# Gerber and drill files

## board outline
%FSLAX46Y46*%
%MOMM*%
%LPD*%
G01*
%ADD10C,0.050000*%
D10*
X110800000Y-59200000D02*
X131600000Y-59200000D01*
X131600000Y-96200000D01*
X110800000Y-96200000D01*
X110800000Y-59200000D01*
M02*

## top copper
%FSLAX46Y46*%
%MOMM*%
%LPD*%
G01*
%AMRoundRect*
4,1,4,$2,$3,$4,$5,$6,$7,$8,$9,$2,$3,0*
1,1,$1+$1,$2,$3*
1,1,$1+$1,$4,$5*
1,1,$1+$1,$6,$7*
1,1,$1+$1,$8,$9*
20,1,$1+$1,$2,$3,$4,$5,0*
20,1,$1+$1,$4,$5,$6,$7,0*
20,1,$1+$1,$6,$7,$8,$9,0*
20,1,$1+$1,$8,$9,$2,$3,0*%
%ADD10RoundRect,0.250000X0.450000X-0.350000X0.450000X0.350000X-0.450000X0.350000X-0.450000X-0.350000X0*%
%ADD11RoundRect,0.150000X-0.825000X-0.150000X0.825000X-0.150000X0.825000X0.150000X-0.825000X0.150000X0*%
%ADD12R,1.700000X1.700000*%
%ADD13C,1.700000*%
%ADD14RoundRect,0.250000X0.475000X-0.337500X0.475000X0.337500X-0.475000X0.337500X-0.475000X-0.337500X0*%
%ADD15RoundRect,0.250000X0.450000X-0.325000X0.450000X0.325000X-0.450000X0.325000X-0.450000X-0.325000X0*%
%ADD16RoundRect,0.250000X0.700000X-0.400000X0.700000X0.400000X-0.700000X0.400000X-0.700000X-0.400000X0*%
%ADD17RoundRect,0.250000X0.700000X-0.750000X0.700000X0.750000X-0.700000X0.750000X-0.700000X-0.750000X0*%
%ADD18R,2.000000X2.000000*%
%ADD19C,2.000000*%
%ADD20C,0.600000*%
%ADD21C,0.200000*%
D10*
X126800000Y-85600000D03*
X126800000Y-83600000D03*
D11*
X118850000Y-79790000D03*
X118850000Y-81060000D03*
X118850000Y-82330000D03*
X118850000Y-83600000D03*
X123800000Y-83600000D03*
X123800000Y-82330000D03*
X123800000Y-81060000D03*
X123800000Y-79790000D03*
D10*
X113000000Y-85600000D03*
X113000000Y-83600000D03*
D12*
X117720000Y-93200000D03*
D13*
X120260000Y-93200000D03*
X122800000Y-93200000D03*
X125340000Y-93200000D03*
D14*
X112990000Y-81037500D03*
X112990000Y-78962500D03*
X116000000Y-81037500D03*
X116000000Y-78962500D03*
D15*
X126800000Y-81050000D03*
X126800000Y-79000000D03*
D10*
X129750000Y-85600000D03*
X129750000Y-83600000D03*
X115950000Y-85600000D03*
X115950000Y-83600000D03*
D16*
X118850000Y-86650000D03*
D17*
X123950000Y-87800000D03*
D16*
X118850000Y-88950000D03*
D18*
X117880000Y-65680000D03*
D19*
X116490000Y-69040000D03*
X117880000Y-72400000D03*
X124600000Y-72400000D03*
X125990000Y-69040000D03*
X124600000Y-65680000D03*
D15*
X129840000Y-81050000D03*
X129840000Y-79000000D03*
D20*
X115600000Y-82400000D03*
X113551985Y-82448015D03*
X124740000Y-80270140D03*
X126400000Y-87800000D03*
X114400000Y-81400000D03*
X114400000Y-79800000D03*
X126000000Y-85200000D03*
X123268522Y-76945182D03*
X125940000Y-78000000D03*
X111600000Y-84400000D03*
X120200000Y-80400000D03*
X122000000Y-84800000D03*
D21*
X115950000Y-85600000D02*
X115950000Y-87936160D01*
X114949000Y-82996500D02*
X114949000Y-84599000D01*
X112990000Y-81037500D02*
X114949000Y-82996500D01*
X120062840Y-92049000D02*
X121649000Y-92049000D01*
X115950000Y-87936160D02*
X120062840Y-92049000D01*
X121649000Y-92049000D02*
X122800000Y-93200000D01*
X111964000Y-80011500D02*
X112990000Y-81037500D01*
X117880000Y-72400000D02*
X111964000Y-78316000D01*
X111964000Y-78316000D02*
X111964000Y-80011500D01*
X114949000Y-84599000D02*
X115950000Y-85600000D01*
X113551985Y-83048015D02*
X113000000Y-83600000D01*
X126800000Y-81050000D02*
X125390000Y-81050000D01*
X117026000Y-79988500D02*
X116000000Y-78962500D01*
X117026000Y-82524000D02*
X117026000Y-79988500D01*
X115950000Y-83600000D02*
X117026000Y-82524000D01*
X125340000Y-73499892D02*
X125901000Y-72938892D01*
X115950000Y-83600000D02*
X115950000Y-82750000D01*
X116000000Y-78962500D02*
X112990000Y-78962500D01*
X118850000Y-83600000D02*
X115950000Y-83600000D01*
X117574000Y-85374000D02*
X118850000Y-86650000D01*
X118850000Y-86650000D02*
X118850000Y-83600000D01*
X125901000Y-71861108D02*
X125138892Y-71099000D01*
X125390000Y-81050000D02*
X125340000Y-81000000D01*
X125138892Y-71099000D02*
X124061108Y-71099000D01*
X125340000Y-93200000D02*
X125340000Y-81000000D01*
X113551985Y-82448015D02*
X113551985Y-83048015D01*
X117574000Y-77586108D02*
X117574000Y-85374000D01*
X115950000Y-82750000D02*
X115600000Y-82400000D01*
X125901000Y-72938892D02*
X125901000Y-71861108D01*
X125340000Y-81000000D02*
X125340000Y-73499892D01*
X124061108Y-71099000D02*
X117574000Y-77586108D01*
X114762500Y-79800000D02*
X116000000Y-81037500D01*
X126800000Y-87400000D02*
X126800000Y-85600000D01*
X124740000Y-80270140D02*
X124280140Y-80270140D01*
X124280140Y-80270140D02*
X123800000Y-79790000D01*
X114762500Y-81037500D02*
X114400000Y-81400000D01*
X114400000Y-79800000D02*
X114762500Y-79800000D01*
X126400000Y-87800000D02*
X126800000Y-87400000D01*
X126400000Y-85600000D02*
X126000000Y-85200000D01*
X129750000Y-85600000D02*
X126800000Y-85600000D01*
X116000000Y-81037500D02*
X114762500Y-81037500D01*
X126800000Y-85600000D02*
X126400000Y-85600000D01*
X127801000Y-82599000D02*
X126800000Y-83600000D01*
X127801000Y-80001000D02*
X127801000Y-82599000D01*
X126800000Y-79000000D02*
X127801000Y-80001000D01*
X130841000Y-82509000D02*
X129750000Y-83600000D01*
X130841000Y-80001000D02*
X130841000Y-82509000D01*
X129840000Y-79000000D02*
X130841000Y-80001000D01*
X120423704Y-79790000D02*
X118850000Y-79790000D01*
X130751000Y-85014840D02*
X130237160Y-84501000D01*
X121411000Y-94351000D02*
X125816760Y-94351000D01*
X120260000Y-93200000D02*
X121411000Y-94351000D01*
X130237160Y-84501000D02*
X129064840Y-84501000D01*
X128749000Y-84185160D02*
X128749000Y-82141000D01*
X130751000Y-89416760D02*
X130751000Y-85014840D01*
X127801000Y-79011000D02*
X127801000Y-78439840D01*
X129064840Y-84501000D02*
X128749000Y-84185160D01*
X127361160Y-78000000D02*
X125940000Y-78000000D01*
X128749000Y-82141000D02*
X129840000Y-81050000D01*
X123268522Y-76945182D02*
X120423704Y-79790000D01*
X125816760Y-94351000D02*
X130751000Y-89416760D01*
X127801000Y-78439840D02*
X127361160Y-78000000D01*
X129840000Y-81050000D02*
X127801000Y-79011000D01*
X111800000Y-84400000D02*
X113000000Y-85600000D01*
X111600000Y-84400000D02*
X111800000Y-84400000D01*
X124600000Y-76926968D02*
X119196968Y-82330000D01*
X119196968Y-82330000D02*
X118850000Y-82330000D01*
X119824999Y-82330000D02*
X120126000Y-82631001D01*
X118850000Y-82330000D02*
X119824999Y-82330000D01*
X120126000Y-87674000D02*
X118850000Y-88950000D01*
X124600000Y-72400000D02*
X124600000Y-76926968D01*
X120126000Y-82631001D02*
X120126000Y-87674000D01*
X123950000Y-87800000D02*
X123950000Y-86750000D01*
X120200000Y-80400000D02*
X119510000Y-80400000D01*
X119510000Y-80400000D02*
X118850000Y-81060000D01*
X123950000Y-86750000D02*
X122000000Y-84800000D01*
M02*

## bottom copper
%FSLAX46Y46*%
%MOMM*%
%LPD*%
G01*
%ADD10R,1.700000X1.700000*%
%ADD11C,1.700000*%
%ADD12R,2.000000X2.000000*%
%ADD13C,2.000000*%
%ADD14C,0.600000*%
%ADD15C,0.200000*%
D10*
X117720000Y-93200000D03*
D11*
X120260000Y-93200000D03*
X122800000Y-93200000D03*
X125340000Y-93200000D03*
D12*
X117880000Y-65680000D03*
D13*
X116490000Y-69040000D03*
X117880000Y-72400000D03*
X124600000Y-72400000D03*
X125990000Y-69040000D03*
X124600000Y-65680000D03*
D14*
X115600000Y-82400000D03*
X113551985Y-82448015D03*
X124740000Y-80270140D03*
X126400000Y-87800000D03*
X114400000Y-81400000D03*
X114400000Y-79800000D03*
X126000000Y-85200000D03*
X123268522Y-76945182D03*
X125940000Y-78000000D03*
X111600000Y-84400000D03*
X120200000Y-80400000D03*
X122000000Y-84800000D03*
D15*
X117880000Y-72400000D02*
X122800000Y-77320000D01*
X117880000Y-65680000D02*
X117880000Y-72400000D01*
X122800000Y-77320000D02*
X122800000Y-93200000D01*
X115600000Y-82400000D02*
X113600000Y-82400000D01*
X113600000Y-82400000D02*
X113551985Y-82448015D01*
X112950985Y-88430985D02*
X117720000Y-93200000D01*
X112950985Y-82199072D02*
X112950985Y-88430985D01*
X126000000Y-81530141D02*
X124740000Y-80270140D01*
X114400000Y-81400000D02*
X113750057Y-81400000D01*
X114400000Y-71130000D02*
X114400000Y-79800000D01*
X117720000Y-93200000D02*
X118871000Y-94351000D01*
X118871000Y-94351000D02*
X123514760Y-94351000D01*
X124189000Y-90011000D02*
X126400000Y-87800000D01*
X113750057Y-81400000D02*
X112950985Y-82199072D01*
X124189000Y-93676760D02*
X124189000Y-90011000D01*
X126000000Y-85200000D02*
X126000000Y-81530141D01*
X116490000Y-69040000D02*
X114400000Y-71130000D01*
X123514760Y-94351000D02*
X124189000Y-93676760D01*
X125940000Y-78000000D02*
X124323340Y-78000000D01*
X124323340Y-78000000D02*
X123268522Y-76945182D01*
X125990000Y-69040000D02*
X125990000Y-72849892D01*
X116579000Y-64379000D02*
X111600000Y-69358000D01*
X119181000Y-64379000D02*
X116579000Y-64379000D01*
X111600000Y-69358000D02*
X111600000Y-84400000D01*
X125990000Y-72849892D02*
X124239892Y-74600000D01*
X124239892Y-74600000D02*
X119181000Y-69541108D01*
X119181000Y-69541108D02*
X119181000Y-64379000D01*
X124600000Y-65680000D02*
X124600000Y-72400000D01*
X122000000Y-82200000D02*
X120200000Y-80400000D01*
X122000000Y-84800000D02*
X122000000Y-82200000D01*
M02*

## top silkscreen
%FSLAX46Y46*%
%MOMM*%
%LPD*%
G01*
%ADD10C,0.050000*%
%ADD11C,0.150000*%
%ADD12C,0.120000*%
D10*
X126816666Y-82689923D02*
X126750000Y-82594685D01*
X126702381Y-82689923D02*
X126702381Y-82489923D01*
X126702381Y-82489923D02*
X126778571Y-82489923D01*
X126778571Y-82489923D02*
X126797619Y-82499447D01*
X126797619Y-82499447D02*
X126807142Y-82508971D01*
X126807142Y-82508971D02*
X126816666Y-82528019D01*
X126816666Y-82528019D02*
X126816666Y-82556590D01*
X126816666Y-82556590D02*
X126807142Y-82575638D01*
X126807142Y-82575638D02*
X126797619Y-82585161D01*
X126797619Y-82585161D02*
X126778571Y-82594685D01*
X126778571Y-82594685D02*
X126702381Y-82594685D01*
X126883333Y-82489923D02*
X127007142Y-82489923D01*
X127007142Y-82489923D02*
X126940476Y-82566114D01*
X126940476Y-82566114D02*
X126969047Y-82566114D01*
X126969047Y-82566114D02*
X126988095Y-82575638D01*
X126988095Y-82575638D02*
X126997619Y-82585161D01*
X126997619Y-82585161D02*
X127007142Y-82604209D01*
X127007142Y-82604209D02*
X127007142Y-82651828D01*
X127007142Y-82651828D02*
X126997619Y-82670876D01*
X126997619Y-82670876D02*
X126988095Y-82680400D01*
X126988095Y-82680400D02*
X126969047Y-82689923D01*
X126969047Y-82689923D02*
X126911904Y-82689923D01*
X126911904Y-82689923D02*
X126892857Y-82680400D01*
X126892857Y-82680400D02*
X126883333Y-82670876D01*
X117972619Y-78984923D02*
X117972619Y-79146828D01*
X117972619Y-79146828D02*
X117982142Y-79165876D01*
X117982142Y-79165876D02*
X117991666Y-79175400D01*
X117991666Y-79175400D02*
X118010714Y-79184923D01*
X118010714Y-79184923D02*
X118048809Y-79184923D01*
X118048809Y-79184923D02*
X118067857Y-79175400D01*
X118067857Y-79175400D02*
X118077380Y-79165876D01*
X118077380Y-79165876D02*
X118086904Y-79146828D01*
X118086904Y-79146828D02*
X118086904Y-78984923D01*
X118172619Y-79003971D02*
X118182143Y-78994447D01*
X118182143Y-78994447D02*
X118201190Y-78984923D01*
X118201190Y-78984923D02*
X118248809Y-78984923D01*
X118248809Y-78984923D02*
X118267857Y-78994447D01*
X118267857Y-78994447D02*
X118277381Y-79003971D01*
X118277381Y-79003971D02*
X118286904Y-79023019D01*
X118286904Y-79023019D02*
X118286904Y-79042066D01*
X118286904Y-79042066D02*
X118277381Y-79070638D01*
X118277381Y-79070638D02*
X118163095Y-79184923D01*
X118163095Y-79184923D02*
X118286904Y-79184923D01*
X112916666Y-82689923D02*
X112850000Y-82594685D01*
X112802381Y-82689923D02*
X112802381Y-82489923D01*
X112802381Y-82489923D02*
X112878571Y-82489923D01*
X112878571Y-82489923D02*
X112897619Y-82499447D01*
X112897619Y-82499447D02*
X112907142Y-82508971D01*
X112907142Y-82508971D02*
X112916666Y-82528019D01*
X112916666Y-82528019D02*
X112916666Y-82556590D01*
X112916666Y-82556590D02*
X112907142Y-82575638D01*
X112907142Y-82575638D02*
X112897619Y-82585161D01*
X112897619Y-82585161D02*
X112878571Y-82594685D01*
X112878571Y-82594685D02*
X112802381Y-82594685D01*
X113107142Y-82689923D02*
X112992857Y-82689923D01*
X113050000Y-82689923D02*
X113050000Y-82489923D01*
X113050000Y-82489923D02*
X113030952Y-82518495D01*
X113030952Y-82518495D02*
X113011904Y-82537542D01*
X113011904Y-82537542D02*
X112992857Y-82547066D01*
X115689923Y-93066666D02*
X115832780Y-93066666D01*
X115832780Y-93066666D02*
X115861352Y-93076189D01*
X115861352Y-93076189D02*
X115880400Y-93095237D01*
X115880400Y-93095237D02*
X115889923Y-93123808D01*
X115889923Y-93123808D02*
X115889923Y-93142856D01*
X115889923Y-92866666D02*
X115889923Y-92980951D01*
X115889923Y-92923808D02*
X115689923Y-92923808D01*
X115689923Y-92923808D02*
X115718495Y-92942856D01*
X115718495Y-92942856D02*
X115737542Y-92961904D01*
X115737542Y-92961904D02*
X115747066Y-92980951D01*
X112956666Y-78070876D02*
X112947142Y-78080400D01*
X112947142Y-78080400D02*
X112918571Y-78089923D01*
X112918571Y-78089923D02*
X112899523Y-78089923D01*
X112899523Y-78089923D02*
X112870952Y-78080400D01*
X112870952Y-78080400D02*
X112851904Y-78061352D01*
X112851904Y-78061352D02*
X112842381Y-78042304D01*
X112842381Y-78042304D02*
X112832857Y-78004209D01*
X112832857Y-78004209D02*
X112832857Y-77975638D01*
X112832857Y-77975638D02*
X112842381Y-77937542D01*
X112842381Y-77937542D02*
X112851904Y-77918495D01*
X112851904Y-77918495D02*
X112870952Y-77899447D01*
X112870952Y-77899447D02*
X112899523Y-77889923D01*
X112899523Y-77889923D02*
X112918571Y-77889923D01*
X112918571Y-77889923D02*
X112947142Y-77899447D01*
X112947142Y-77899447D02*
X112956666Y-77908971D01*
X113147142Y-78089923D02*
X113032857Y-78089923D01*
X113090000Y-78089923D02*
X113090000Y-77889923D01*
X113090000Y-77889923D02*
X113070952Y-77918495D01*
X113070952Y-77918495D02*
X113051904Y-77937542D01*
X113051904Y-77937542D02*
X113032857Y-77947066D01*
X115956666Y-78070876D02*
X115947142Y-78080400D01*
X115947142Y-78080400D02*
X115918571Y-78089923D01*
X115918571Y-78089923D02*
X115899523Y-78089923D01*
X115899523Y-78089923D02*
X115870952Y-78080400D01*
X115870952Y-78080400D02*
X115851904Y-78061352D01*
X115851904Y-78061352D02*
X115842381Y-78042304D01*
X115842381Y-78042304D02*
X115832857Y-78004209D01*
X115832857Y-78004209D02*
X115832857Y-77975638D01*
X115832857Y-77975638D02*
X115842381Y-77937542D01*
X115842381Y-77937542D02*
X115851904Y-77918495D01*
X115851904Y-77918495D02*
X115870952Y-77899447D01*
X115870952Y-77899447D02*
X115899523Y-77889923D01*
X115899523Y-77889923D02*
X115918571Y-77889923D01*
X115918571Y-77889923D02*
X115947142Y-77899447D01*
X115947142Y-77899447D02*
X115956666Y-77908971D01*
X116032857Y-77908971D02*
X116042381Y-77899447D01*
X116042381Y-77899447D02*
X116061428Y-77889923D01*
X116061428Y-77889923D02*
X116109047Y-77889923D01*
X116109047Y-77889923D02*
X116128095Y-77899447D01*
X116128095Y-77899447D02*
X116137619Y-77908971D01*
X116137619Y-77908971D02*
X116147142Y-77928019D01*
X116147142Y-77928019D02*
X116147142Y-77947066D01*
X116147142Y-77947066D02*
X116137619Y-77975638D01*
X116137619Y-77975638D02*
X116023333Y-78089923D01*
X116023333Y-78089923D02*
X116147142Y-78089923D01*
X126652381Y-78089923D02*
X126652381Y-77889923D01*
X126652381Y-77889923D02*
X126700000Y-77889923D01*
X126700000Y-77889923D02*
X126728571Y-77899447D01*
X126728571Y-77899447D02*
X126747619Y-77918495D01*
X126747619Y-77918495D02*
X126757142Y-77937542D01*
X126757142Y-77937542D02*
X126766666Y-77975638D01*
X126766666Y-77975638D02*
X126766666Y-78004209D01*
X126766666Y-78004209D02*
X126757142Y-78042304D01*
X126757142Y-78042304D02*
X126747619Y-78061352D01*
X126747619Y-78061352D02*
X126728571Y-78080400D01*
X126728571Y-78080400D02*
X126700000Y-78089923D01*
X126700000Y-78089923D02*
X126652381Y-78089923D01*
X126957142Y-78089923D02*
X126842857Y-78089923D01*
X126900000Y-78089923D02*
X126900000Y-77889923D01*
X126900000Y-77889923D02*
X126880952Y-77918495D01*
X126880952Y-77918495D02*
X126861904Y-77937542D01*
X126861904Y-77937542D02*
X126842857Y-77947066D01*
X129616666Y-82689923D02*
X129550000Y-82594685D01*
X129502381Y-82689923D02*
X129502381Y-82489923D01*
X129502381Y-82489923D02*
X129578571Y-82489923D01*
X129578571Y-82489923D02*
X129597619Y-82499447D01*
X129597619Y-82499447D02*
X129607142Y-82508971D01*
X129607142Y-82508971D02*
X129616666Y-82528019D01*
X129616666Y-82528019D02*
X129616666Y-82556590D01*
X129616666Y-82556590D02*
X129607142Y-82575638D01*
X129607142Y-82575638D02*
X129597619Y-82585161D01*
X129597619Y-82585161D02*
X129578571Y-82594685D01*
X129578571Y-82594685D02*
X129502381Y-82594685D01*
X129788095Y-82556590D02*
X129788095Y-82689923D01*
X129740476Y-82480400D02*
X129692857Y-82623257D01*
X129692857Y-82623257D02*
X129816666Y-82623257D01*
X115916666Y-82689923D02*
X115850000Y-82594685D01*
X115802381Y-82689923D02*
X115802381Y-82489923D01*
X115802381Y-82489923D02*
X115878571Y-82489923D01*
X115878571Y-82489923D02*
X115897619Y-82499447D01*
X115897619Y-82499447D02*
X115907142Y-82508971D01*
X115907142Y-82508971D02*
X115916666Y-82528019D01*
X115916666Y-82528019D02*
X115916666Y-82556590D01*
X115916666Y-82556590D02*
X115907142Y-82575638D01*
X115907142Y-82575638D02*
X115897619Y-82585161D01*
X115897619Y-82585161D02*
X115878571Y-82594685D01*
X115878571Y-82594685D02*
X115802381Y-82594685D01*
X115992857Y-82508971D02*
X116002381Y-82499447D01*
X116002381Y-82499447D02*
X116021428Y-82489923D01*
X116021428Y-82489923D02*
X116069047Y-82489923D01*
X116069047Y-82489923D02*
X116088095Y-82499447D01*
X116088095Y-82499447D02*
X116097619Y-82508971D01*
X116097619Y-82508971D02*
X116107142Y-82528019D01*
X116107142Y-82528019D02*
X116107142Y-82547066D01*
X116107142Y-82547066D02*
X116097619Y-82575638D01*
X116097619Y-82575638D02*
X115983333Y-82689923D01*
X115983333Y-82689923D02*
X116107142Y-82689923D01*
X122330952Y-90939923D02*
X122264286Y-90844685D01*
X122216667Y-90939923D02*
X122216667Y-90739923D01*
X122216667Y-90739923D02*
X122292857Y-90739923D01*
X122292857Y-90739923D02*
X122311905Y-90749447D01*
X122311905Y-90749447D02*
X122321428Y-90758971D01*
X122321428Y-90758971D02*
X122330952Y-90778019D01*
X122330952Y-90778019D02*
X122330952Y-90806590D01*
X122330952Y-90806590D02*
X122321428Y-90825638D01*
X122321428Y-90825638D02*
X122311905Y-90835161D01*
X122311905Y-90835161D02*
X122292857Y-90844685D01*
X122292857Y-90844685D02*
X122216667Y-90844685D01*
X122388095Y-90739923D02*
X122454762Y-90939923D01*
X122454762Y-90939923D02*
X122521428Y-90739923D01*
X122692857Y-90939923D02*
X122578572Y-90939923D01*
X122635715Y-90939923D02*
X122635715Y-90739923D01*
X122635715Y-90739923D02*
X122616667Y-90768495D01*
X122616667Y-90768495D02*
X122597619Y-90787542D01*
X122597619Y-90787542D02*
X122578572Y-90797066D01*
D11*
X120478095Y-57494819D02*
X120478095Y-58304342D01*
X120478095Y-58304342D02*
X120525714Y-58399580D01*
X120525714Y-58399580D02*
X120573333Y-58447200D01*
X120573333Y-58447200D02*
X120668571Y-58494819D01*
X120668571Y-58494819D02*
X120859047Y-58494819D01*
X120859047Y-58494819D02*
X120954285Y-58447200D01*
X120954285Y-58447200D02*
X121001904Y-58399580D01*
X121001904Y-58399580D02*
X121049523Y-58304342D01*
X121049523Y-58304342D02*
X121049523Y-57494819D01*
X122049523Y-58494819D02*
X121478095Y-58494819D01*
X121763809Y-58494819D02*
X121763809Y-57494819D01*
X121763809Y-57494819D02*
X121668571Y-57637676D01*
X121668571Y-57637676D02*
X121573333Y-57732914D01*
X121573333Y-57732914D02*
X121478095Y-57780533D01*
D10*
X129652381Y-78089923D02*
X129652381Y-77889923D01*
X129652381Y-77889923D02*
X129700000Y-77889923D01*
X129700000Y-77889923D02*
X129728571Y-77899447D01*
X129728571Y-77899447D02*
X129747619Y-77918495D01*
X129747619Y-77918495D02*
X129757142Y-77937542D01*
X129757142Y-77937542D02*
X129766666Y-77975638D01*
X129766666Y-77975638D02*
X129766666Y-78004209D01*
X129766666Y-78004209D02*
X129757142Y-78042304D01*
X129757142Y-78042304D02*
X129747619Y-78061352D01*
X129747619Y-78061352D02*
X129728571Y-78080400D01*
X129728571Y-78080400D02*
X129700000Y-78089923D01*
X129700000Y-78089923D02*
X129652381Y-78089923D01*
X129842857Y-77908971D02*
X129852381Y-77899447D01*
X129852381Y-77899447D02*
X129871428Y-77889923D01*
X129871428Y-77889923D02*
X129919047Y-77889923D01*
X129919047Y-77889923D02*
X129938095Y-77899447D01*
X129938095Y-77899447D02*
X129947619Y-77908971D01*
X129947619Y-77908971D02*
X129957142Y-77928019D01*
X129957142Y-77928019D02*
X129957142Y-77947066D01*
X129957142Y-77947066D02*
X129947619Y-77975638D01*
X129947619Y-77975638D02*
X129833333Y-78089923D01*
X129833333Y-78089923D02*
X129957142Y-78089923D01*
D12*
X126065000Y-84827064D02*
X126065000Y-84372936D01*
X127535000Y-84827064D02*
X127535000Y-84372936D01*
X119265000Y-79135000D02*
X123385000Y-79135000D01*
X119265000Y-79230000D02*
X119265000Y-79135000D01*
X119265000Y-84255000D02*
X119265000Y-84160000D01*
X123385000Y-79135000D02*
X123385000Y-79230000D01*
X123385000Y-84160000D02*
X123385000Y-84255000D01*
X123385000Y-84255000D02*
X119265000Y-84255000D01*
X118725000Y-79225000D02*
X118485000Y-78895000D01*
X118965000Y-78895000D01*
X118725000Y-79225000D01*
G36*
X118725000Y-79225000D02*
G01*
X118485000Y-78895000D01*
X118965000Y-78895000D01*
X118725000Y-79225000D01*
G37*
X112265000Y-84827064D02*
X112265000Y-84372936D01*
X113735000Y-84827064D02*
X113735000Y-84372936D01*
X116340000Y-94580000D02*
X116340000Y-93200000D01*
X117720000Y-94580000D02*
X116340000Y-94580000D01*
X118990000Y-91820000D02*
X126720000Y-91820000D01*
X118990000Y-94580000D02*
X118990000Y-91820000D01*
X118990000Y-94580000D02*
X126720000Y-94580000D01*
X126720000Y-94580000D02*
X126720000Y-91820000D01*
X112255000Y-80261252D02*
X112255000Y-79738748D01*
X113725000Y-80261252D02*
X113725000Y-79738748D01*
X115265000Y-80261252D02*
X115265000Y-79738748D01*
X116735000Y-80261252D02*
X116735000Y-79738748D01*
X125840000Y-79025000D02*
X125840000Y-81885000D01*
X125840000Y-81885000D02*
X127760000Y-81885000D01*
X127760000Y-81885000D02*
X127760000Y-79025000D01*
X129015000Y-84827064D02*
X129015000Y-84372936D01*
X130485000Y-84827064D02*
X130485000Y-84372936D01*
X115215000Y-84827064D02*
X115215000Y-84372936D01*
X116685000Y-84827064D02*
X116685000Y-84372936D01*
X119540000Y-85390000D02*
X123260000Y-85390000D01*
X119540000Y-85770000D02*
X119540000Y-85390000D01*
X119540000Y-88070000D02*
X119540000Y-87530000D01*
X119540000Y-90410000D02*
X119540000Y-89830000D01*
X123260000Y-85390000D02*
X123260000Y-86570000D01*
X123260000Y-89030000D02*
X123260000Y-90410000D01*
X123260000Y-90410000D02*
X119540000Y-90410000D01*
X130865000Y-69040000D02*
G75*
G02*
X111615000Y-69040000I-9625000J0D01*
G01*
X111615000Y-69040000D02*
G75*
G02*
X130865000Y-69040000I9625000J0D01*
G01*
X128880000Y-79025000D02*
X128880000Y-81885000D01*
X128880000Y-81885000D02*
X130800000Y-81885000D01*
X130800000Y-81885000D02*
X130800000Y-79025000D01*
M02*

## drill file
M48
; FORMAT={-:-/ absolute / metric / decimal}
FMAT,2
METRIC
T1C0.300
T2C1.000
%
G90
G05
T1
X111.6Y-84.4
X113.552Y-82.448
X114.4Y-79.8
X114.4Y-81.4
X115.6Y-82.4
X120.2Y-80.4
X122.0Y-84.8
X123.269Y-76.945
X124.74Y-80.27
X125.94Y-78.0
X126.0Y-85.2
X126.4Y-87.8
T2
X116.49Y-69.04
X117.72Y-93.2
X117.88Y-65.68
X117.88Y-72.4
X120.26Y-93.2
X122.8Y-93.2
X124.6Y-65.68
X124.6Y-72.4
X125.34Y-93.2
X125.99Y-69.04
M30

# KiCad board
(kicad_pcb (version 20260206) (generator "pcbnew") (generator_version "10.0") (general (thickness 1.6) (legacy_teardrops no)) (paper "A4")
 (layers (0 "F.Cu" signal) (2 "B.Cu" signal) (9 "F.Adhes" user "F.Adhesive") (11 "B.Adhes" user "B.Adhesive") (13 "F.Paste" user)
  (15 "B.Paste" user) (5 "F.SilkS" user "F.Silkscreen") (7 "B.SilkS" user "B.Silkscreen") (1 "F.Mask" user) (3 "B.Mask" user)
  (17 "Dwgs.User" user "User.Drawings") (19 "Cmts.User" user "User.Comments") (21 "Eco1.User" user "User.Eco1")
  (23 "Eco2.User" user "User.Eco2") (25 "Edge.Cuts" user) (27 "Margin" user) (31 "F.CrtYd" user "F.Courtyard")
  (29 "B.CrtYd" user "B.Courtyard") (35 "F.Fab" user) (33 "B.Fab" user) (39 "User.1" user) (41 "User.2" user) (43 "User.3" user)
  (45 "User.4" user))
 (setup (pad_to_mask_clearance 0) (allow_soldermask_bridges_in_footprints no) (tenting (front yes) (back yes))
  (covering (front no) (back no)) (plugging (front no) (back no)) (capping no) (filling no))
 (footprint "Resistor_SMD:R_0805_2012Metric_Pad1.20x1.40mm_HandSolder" (layer "F.Cu") (at 126.8 84.6 90)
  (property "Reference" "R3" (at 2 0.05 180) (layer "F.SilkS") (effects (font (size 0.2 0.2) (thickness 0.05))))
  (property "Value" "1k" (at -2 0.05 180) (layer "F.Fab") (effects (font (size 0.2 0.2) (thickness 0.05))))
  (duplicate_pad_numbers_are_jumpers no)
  (fp_line (start -0.227064 -0.735) (end 0.227064 -0.735) (stroke (width 0.12) (type solid)) (layer "F.SilkS"))
  (fp_line (start -0.227064 0.735) (end 0.227064 0.735) (stroke (width 0.12) (type solid)) (layer "F.SilkS"))
  (pad "1" smd roundrect (at -1 0 90) (size 1.2 1.4) (layers "F.Cu" "F.Mask" "F.Paste") (roundrect_rratio 0.208333) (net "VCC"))
  (pad "2" smd roundrect (at 1 0 90) (size 1.2 1.4) (layers "F.Cu" "F.Mask" "F.Paste") (roundrect_rratio 0.208333) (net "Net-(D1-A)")))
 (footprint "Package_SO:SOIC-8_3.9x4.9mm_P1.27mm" (layer "F.Cu") (at 121.325 81.695)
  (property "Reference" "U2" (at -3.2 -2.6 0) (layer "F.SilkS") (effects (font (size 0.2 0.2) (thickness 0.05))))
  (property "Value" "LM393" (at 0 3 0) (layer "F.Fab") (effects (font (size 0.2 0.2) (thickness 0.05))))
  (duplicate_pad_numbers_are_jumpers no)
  (fp_line (start -2.06 -2.56) (end 2.06 -2.56) (stroke (width 0.12) (type solid)) (layer "F.SilkS"))
  (fp_line (start -2.06 -2.465) (end -2.06 -2.56) (stroke (width 0.12) (type solid)) (layer "F.SilkS"))
  (fp_line (start -2.06 2.56) (end -2.06 2.465) (stroke (width 0.12) (type solid)) (layer "F.SilkS"))
  (fp_line (start 2.06 -2.56) (end 2.06 -2.465) (stroke (width 0.12) (type solid)) (layer "F.SilkS"))
  (fp_line (start 2.06 2.465) (end 2.06 2.56) (stroke (width 0.12) (type solid)) (layer "F.SilkS"))
  (fp_line (start 2.06 2.56) (end -2.06 2.56) (stroke (width 0.12) (type solid)) (layer "F.SilkS"))
  (fp_poly (pts (xy -2.6 -2.47) (xy -2.84 -2.8) (xy -2.36 -2.8)) (stroke (width 0.12) (type solid)) (fill yes) (layer "F.SilkS"))
  (pad "1" smd roundrect (at -2.475 -1.905) (size 1.95 0.6) (layers "F.Cu" "F.Mask" "F.Paste") (roundrect_rratio 0.25) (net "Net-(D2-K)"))
  (pad "2" smd roundrect (at -2.475 -0.635) (size 1.95 0.6) (layers "F.Cu" "F.Mask" "F.Paste") (roundrect_rratio 0.25) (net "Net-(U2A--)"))
  (pad "3" smd roundrect (at -2.475 0.635) (size 1.95 0.6) (layers "F.Cu" "F.Mask" "F.Paste") (roundrect_rratio 0.25) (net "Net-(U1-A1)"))
  (pad "4" smd roundrect (at -2.475 1.905) (size 1.95 0.6) (layers "F.Cu" "F.Mask" "F.Paste") (roundrect_rratio 0.25) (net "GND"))
  (pad "5" smd roundrect (at 2.475 1.905) (size 1.95 0.6) (layers "F.Cu" "F.Mask" "F.Paste") (roundrect_rratio 0.25))
  (pad "6" smd roundrect (at 2.475 0.635) (size 1.95 0.6) (layers "F.Cu" "F.Mask" "F.Paste") (roundrect_rratio 0.25))
  (pad "7" smd roundrect (at 2.475 -0.635) (size 1.95 0.6) (layers "F.Cu" "F.Mask" "F.Paste") (roundrect_rratio 0.25))
  (pad "8" smd roundrect (at 2.475 -1.905) (size 1.95 0.6) (layers "F.Cu" "F.Mask" "F.Paste") (roundrect_rratio 0.25) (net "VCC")))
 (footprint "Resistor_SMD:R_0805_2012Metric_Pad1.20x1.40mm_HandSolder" (layer "F.Cu") (at 113 84.6 90)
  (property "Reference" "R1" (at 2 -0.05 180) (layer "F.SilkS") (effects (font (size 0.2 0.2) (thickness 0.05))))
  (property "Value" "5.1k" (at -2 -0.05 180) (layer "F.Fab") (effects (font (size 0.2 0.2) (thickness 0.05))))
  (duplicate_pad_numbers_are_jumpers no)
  (fp_line (start -0.227064 -0.735) (end 0.227064 -0.735) (stroke (width 0.12) (type solid)) (layer "F.SilkS"))
  (fp_line (start -0.227064 0.735) (end 0.227064 0.735) (stroke (width 0.12) (type solid)) (layer "F.SilkS"))
  (pad "1" smd roundrect (at -1 0 90) (size 1.2 1.4) (layers "F.Cu" "F.Mask" "F.Paste") (roundrect_rratio 0.208333) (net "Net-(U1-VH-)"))
  (pad "2" smd roundrect (at 1 0 90) (size 1.2 1.4) (layers "F.Cu" "F.Mask" "F.Paste") (roundrect_rratio 0.208333) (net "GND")))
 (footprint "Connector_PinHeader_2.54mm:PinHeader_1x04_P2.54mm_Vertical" (layer "F.Cu") (at 117.72 93.2 90)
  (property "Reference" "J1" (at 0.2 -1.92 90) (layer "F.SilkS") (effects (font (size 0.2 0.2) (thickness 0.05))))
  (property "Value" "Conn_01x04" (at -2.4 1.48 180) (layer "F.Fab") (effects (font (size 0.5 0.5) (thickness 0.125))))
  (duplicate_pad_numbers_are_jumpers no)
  (fp_line (start -1.38 -1.38) (end 0 -1.38) (stroke (width 0.12) (type solid)) (layer "F.SilkS"))
  (fp_line (start -1.38 0) (end -1.38 -1.38) (stroke (width 0.12) (type solid)) (layer "F.SilkS"))
  (fp_line (start 1.38 1.27) (end 1.38 9) (stroke (width 0.12) (type solid)) (layer "F.SilkS"))
  (fp_line (start -1.38 1.27) (end 1.38 1.27) (stroke (width 0.12) (type solid)) (layer "F.SilkS"))
  (fp_line (start -1.38 1.27) (end -1.38 9) (stroke (width 0.12) (type solid)) (layer "F.SilkS"))
  (fp_line (start -1.38 9) (end 1.38 9) (stroke (width 0.12) (type solid)) (layer "F.SilkS"))
  (pad "1" thru_hole rect (at 0 0 90) (size 1.7 1.7) (drill 1) (layers "*.Cu" "*.Mask") (remove_unused_layers no) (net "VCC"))
  (pad "2" thru_hole circle (at 0 2.54 90) (size 1.7 1.7) (drill 1) (layers "*.Cu" "*.Mask") (remove_unused_layers no) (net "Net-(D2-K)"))
  (pad "3" thru_hole circle (at 0 5.08 90) (size 1.7 1.7) (drill 1) (layers "*.Cu" "*.Mask") (remove_unused_layers no)
   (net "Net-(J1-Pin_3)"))
  (pad "4" thru_hole circle (at 0 7.62 90) (size 1.7 1.7) (drill 1) (layers "*.Cu" "*.Mask") (remove_unused_layers no) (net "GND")))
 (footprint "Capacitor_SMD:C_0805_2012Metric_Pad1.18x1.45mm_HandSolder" (layer "F.Cu") (at 112.99 80 90)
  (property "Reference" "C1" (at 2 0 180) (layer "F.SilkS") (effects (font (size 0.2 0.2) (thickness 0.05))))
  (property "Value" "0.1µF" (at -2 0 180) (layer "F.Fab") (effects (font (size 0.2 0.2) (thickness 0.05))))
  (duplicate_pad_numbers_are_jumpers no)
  (fp_line (start -0.261252 -0.735) (end 0.261252 -0.735) (stroke (width 0.12) (type solid)) (layer "F.SilkS"))
  (fp_line (start -0.261252 0.735) (end 0.261252 0.735) (stroke (width 0.12) (type solid)) (layer "F.SilkS"))
  (pad "1" smd roundrect (at -1.0375 0 90) (size 1.175 1.45) (layers "F.Cu" "F.Mask" "F.Paste") (roundrect_rratio 0.212766)
   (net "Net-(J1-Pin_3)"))
  (pad "2" smd roundrect (at 1.0375 0 90) (size 1.175 1.45) (layers "F.Cu" "F.Mask" "F.Paste") (roundrect_rratio 0.212766) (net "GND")))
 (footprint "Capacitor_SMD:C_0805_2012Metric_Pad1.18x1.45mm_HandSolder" (layer "F.Cu") (at 116 80 90)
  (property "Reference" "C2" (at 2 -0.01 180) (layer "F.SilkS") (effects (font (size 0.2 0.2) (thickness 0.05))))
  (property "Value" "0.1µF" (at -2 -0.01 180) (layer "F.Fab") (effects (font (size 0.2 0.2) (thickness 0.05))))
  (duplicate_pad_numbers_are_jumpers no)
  (fp_line (start -0.261252 -0.735) (end 0.261252 -0.735) (stroke (width 0.12) (type solid)) (layer "F.SilkS"))
  (fp_line (start -0.261252 0.735) (end 0.261252 0.735) (stroke (width 0.12) (type solid)) (layer "F.SilkS"))
  (pad "1" smd roundrect (at -1.0375 0 90) (size 1.175 1.45) (layers "F.Cu" "F.Mask" "F.Paste") (roundrect_rratio 0.212766) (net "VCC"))
  (pad "2" smd roundrect (at 1.0375 0 90) (size 1.175 1.45) (layers "F.Cu" "F.Mask" "F.Paste") (roundrect_rratio 0.212766) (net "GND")))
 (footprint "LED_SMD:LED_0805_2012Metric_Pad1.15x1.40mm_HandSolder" (layer "F.Cu") (at 126.8 80.025 90)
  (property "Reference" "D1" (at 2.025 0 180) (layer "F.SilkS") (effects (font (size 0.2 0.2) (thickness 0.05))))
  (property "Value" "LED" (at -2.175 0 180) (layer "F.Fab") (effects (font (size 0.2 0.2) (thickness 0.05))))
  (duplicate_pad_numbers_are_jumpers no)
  (fp_line (start 1 -0.96) (end -1.86 -0.96) (stroke (width 0.12) (type solid)) (layer "F.SilkS"))
  (fp_line (start -1.86 -0.96) (end -1.86 0.96) (stroke (width 0.12) (type solid)) (layer "F.SilkS"))
  (fp_line (start -1.86 0.96) (end 1 0.96) (stroke (width 0.12) (type solid)) (layer "F.SilkS"))
  (pad "1" smd roundrect (at -1.025 0 90) (size 1.15 1.4) (layers "F.Cu" "F.Mask" "F.Paste") (roundrect_rratio 0.217391) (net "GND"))
  (pad "2" smd roundrect (at 1.025 0 90) (size 1.15 1.4) (layers "F.Cu" "F.Mask" "F.Paste") (roundrect_rratio 0.217391) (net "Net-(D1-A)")))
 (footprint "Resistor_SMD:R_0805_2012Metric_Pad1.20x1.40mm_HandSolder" (layer "F.Cu") (at 129.75 84.6 90)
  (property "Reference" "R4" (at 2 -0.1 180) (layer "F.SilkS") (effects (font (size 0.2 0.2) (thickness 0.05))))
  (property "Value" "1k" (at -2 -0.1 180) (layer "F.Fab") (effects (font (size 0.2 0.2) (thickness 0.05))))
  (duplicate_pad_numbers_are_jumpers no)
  (fp_line (start -0.227064 -0.735) (end 0.227064 -0.735) (stroke (width 0.12) (type solid)) (layer "F.SilkS"))
  (fp_line (start -0.227064 0.735) (end 0.227064 0.735) (stroke (width 0.12) (type solid)) (layer "F.SilkS"))
  (pad "1" smd roundrect (at -1 0 90) (size 1.2 1.4) (layers "F.Cu" "F.Mask" "F.Paste") (roundrect_rratio 0.208333) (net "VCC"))
  (pad "2" smd roundrect (at 1 0 90) (size 1.2 1.4) (layers "F.Cu" "F.Mask" "F.Paste") (roundrect_rratio 0.208333) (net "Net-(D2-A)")))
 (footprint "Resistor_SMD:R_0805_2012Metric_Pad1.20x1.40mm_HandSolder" (layer "F.Cu") (at 115.95 84.6 90)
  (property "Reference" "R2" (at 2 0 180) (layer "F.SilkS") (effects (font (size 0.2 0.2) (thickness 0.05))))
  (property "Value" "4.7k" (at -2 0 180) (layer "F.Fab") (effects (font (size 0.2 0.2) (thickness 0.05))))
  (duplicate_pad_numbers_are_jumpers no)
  (fp_line (start -0.227064 -0.735) (end 0.227064 -0.735) (stroke (width 0.12) (type solid)) (layer "F.SilkS"))
  (fp_line (start -0.227064 0.735) (end 0.227064 0.735) (stroke (width 0.12) (type solid)) (layer "F.SilkS"))
  (pad "1" smd roundrect (at -1 0 90) (size 1.2 1.4) (layers "F.Cu" "F.Mask" "F.Paste") (roundrect_rratio 0.208333) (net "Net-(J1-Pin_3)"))
  (pad "2" smd roundrect (at 1 0 90) (size 1.2 1.4) (layers "F.Cu" "F.Mask" "F.Paste") (roundrect_rratio 0.208333) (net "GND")))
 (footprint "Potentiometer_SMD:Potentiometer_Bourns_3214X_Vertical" (layer "F.Cu") (at 121.4 87.8 90)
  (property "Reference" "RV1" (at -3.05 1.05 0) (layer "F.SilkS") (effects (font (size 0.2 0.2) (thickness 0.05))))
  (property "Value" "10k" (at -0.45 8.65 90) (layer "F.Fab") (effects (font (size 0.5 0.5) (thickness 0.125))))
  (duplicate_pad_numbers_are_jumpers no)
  (fp_line (start 2.41 -1.86) (end 2.41 1.86) (stroke (width 0.12) (type solid)) (layer "F.SilkS"))
  (fp_line (start 2.03 -1.86) (end 2.41 -1.86) (stroke (width 0.12) (type solid)) (layer "F.SilkS"))
  (fp_line (start -0.27 -1.86) (end 0.27 -1.86) (stroke (width 0.12) (type solid)) (layer "F.SilkS"))
  (fp_line (start -2.61 -1.86) (end -2.03 -1.86) (stroke (width 0.12) (type solid)) (layer "F.SilkS"))
  (fp_line (start 2.41 1.86) (end 1.23 1.86) (stroke (width 0.12) (type solid)) (layer "F.SilkS"))
  (fp_line (start -1.23 1.86) (end -2.61 1.86) (stroke (width 0.12) (type solid)) (layer "F.SilkS"))
  (fp_line (start -2.61 1.86) (end -2.61 -1.86) (stroke (width 0.12) (type solid)) (layer "F.SilkS"))
  (pad "1" smd roundrect (at 1.15 -2.55 90) (size 1.3 1.9) (layers "F.Cu" "F.Mask" "F.Paste") (roundrect_rratio 0.192308) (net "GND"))
  (pad "2" smd roundrect (at 0 2.55 90) (size 2 1.9) (layers "F.Cu" "F.Mask" "F.Paste") (roundrect_rratio 0.131579) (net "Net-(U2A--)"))
  (pad "3" smd roundrect (at -1.15 -2.55 90) (size 1.3 1.9) (layers "F.Cu" "F.Mask" "F.Paste") (roundrect_rratio 0.192308)
   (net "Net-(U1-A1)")))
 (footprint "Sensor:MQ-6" (layer "F.Cu") (at 117.88 65.68)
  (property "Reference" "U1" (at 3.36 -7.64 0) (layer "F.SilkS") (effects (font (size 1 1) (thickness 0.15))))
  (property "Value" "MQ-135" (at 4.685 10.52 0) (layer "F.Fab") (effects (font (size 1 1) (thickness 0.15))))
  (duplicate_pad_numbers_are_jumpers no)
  (fp_circle (center 3.36 3.36) (end 12.985 3.36) (stroke (width 0.12) (type solid)) (fill no) (layer "F.SilkS"))
  (pad "1" thru_hole rect (at 0 0) (size 2 2) (drill 1) (layers "*.Cu" "*.Mask") (remove_unused_layers no) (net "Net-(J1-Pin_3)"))
  (pad "2" thru_hole circle (at -1.39 3.36) (size 2 2) (drill 1) (layers "*.Cu" "*.Mask") (remove_unused_layers no) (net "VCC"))
  (pad "3" thru_hole circle (at 0 6.72 90) (size 2 2) (drill 1) (layers "*.Cu" "*.Mask") (remove_unused_layers no) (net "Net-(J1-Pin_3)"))
  (pad "4" thru_hole circle (at 6.72 6.72 180) (size 2 2) (drill 1) (layers "*.Cu" "*.Mask") (remove_unused_layers no) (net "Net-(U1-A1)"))
  (pad "5" thru_hole circle (at 8.11 3.36) (size 2 2) (drill 1) (layers "*.Cu" "*.Mask") (remove_unused_layers no) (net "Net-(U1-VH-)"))
  (pad "6" thru_hole circle (at 6.72 0 270) (size 2 2) (drill 1) (layers "*.Cu" "*.Mask") (remove_unused_layers no) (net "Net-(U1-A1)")))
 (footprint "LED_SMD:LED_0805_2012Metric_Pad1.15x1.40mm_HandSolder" (layer "F.Cu") (at 129.84 80.025 90)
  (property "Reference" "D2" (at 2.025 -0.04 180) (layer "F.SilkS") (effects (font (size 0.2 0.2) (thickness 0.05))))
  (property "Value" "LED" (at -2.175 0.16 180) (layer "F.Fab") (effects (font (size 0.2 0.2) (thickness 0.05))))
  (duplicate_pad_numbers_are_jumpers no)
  (fp_line (start 1 -0.96) (end -1.86 -0.96) (stroke (width 0.12) (type solid)) (layer "F.SilkS"))
  (fp_line (start -1.86 -0.96) (end -1.86 0.96) (stroke (width 0.12) (type solid)) (layer "F.SilkS"))
  (fp_line (start -1.86 0.96) (end 1 0.96) (stroke (width 0.12) (type solid)) (layer "F.SilkS"))
  (pad "1" smd roundrect (at -1.025 0 90) (size 1.15 1.4) (layers "F.Cu" "F.Mask" "F.Paste") (roundrect_rratio 0.217391) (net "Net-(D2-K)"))
  (pad "2" smd roundrect (at 1.025 0 90) (size 1.15 1.4) (layers "F.Cu" "F.Mask" "F.Paste") (roundrect_rratio 0.217391) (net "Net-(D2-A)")))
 (gr_rect (start 110.8 59.2) (end 131.6 96.2) (stroke (width 0.05) (type default)) (fill no) (layer "Edge.Cuts"))
 (segment (start 115.95 85.6) (end 115.95 87.93616) (width 0.2) (layer "F.Cu") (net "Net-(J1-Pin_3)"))
 (segment (start 114.949 82.9965) (end 114.949 84.599) (width 0.2) (layer "F.Cu") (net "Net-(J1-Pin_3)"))
 (segment (start 112.99 81.0375) (end 114.949 82.9965) (width 0.2) (layer "F.Cu") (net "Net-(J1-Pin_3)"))
 (segment (start 120.06284 92.049) (end 121.649 92.049) (width 0.2) (layer "F.Cu") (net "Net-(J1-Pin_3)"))
 (segment (start 115.95 87.93616) (end 120.06284 92.049) (width 0.2) (layer "F.Cu") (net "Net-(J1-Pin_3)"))
 (segment (start 121.649 92.049) (end 122.8 93.2) (width 0.2) (layer "F.Cu") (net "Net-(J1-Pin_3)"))
 (segment (start 111.964 80.0115) (end 112.99 81.0375) (width 0.2) (layer "F.Cu") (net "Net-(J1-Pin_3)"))
 (segment (start 117.88 72.4) (end 111.964 78.316) (width 0.2) (layer "F.Cu") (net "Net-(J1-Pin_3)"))
 (segment (start 111.964 78.316) (end 111.964 80.0115) (width 0.2) (layer "F.Cu") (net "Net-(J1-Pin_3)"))
 (segment (start 114.949 84.599) (end 115.95 85.6) (width 0.2) (layer "F.Cu") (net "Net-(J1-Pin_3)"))
 (segment (start 117.88 72.4) (end 122.8 77.32) (width 0.2) (layer "B.Cu") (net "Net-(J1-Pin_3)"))
 (segment (start 117.88 65.68) (end 117.88 72.4) (width 0.2) (layer "B.Cu") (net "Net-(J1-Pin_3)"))
 (segment (start 122.8 77.32) (end 122.8 93.2) (width 0.2) (layer "B.Cu") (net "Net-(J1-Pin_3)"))
 (segment (start 113.551985 83.048015) (end 113 83.6) (width 0.2) (layer "F.Cu") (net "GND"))
 (segment (start 126.8 81.05) (end 125.39 81.05) (width 0.2) (layer "F.Cu") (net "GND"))
 (segment (start 117.026 79.9885) (end 116 78.9625) (width 0.2) (layer "F.Cu") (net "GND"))
 (segment (start 117.026 82.524) (end 117.026 79.9885) (width 0.2) (layer "F.Cu") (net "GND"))
 (segment (start 115.95 83.6) (end 117.026 82.524) (width 0.2) (layer "F.Cu") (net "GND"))
 (segment (start 125.34 73.499892) (end 125.901 72.938892) (width 0.2) (layer "F.Cu") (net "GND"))
 (segment (start 115.95 83.6) (end 115.95 82.75) (width 0.2) (layer "F.Cu") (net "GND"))
 (segment (start 116 78.9625) (end 112.99 78.9625) (width 0.2) (layer "F.Cu") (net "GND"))
 (segment (start 118.85 83.6) (end 115.95 83.6) (width 0.2) (layer "F.Cu") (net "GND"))
 (segment (start 117.574 85.374) (end 118.85 86.65) (width 0.2) (layer "F.Cu") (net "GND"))
 (segment (start 118.85 86.65) (end 118.85 83.6) (width 0.2) (layer "F.Cu") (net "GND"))
 (segment (start 125.901 71.861108) (end 125.138892 71.099) (width 0.2) (layer "F.Cu") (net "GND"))
 (segment (start 125.39 81.05) (end 125.34 81) (width 0.2) (layer "F.Cu") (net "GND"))
 (segment (start 125.138892 71.099) (end 124.061108 71.099) (width 0.2) (layer "F.Cu") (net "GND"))
 (segment (start 125.34 93.2) (end 125.34 81) (width 0.2) (layer "F.Cu") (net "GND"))
 (segment (start 113.551985 82.448015) (end 113.551985 83.048015) (width 0.2) (layer "F.Cu") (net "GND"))
 (segment (start 117.574 77.586108) (end 117.574 85.374) (width 0.2) (layer "F.Cu") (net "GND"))
 (segment (start 115.95 82.75) (end 115.6 82.4) (width 0.2) (layer "F.Cu") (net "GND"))
 (segment (start 125.901 72.938892) (end 125.901 71.861108) (width 0.2) (layer "F.Cu") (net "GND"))
 (segment (start 125.34 81) (end 125.34 73.499892) (width 0.2) (layer "F.Cu") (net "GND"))
 (segment (start 124.061108 71.099) (end 117.574 77.586108) (width 0.2) (layer "F.Cu") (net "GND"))
 (via (at 115.6 82.4) (size 0.6) (drill 0.3) (layers "F.Cu" "B.Cu") (capping no) (covering (front no) (back no))
  (plugging (front no) (back no)) (filling no) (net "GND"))
 (via (at 113.551985 82.448015) (size 0.6) (drill 0.3) (layers "F.Cu" "B.Cu") (capping no) (covering (front no) (back no))
  (plugging (front no) (back no)) (filling no) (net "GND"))
 (segment (start 115.6 82.4) (end 113.6 82.4) (width 0.2) (layer "B.Cu") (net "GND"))
 (segment (start 113.6 82.4) (end 113.551985 82.448015) (width 0.2) (layer "B.Cu") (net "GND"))
 (segment (start 114.7625 79.8) (end 116 81.0375) (width 0.2) (layer "F.Cu") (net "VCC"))
 (segment (start 126.8 87.4) (end 126.8 85.6) (width 0.2) (layer "F.Cu") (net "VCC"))
 (segment (start 124.74 80.27014) (end 124.28014 80.27014) (width 0.2) (layer "F.Cu") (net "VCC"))
 (segment (start 124.28014 80.27014) (end 123.8 79.79) (width 0.2) (layer "F.Cu") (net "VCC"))
 (segment (start 114.7625 81.0375) (end 114.4 81.4) (width 0.2) (layer "F.Cu") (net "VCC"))
 (segment (start 114.4 79.8) (end 114.7625 79.8) (width 0.2) (layer "F.Cu") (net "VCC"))
 (segment (start 126.4 87.8) (end 126.8 87.4) (width 0.2) (layer "F.Cu") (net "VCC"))
 (segment (start 126.4 85.6) (end 126 85.2) (width 0.2) (layer "F.Cu") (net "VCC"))
 (segment (start 129.75 85.6) (end 126.8 85.6) (width 0.2) (layer "F.Cu") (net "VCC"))
 (segment (start 116 81.0375) (end 114.7625 81.0375) (width 0.2) (layer "F.Cu") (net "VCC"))
 (segment (start 126.8 85.6) (end 126.4 85.6) (width 0.2) (layer "F.Cu") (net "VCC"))
 (via (at 124.74 80.27014) (size 0.6) (drill 0.3) (layers "F.Cu" "B.Cu") (capping no) (covering (front no) (back no))
  (plugging (front no) (back no)) (filling no) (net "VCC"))
 (via (at 126.4 87.8) (size 0.6) (drill 0.3) (layers "F.Cu" "B.Cu") (capping no) (covering (front no) (back no))
  (plugging (front no) (back no)) (filling no) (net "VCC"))
 (via (at 114.4 81.4) (size 0.6) (drill 0.3) (layers "F.Cu" "B.Cu") (capping no) (covering (front no) (back no))
  (plugging (front no) (back no)) (filling no) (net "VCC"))
 (via (at 114.4 79.8) (size 0.6) (drill 0.3) (layers "F.Cu" "B.Cu") (capping no) (covering (front no) (back no))
  (plugging (front no) (back no)) (filling no) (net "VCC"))
 (via (at 126 85.2) (size 0.6) (drill 0.3) (layers "F.Cu" "B.Cu") (capping no) (covering (front no) (back no))
  (plugging (front no) (back no)) (filling no) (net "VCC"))
 (segment (start 112.950985 88.430985) (end 117.72 93.2) (width 0.2) (layer "B.Cu") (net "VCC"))
 (segment (start 112.950985 82.199072) (end 112.950985 88.430985) (width 0.2) (layer "B.Cu") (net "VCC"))
 (segment (start 126 81.530141) (end 124.74 80.27014) (width 0.2) (layer "B.Cu") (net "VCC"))
 (segment (start 114.4 81.4) (end 113.750057 81.4) (width 0.2) (layer "B.Cu") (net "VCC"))
 (segment (start 114.4 71.13) (end 114.4 79.8) (width 0.2) (layer "B.Cu") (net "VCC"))
 (segment (start 117.72 93.2) (end 118.871 94.351) (width 0.2) (layer "B.Cu") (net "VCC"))
 (segment (start 118.871 94.351) (end 123.51476 94.351) (width 0.2) (layer "B.Cu") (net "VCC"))
 (segment (start 124.189 90.011) (end 126.4 87.8) (width 0.2) (layer "B.Cu") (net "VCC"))
 (segment (start 113.750057 81.4) (end 112.950985 82.199072) (width 0.2) (layer "B.Cu") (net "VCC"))
 (segment (start 124.189 93.67676) (end 124.189 90.011) (width 0.2) (layer "B.Cu") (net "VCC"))
 (segment (start 126 85.2) (end 126 81.530141) (width 0.2) (layer "B.Cu") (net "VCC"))
 (segment (start 116.49 69.04) (end 114.4 71.13) (width 0.2) (layer "B.Cu") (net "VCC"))
 (segment (start 123.51476 94.351) (end 124.189 93.67676) (width 0.2) (layer "B.Cu") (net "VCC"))
 (segment (start 127.801 82.599) (end 126.8 83.6) (width 0.2) (layer "F.Cu") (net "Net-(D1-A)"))
 (segment (start 127.801 80.001) (end 127.801 82.599) (width 0.2) (layer "F.Cu") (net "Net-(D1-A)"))
 (segment (start 126.8 79) (end 127.801 80.001) (width 0.2) (layer "F.Cu") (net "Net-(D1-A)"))
 (segment (start 130.841 82.509) (end 129.75 83.6) (width 0.2) (layer "F.Cu") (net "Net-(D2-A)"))
 (segment (start 130.841 80.001) (end 130.841 82.509) (width 0.2) (layer "F.Cu") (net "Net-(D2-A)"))
 (segment (start 129.84 79) (end 130.841 80.001) (width 0.2) (layer "F.Cu") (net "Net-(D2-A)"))
 (segment (start 120.423704 79.79) (end 118.85 79.79) (width 0.2) (layer "F.Cu") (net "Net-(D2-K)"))
 (segment (start 130.751 85.01484) (end 130.23716 84.501) (width 0.2) (layer "F.Cu") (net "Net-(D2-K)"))
 (segment (start 121.411 94.351) (end 125.81676 94.351) (width 0.2) (layer "F.Cu") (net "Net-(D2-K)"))
 (segment (start 120.26 93.2) (end 121.411 94.351) (width 0.2) (layer "F.Cu") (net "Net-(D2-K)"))
 (segment (start 130.23716 84.501) (end 129.06484 84.501) (width 0.2) (layer "F.Cu") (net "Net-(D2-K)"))
 (segment (start 128.749 84.18516) (end 128.749 82.141) (width 0.2) (layer "F.Cu") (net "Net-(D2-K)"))
 (segment (start 130.751 89.41676) (end 130.751 85.01484) (width 0.2) (layer "F.Cu") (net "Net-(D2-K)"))
 (segment (start 127.801 79.011) (end 127.801 78.43984) (width 0.2) (layer "F.Cu") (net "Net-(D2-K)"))
 (segment (start 129.06484 84.501) (end 128.749 84.18516) (width 0.2) (layer "F.Cu") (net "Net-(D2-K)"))
 (segment (start 127.36116 78) (end 125.94 78) (width 0.2) (layer "F.Cu") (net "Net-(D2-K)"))
 (segment (start 128.749 82.141) (end 129.84 81.05) (width 0.2) (layer "F.Cu") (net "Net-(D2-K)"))
 (segment (start 123.268522 76.945182) (end 120.423704 79.79) (width 0.2) (layer "F.Cu") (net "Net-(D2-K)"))
 (segment (start 125.81676 94.351) (end 130.751 89.41676) (width 0.2) (layer "F.Cu") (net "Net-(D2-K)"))
 (segment (start 127.801 78.43984) (end 127.36116 78) (width 0.2) (layer "F.Cu") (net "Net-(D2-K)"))
 (segment (start 129.84 81.05) (end 127.801 79.011) (width 0.2) (layer "F.Cu") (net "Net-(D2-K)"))
 (via (at 123.268522 76.945182) (size 0.6) (drill 0.3) (layers "F.Cu" "B.Cu") (capping no) (covering (front no) (back no))
  (plugging (front no) (back no)) (filling no) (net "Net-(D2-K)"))
 (via (at 125.94 78) (size 0.6) (drill 0.3) (layers "F.Cu" "B.Cu") (capping no) (covering (front no) (back no))
  (plugging (front no) (back no)) (filling no) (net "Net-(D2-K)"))
 (segment (start 125.94 78) (end 124.32334 78) (width 0.2) (layer "B.Cu") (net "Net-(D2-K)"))
 (segment (start 124.32334 78) (end 123.268522 76.945182) (width 0.2) (layer "B.Cu") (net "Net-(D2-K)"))
 (segment (start 111.8 84.4) (end 113 85.6) (width 0.2) (layer "F.Cu") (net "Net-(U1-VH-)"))
 (segment (start 111.6 84.4) (end 111.8 84.4) (width 0.2) (layer "F.Cu") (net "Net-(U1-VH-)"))
 (via (at 111.6 84.4) (size 0.6) (drill 0.3) (layers "F.Cu" "B.Cu") (capping no) (covering (front no) (back no))
  (plugging (front no) (back no)) (filling no) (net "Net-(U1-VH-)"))
 (segment (start 125.99 69.04) (end 125.99 72.849892) (width 0.2) (layer "B.Cu") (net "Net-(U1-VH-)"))
 (segment (start 116.579 64.379) (end 111.6 69.358) (width 0.2) (layer "B.Cu") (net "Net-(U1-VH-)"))
 (segment (start 119.181 64.379) (end 116.579 64.379) (width 0.2) (layer "B.Cu") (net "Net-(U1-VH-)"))
 (segment (start 111.6 69.358) (end 111.6 84.4) (width 0.2) (layer "B.Cu") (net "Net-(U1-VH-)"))
 (segment (start 125.99 72.849892) (end 124.239892 74.6) (width 0.2) (layer "B.Cu") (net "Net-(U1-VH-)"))
 (segment (start 124.239892 74.6) (end 119.181 69.541108) (width 0.2) (layer "B.Cu") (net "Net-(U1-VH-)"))
 (segment (start 119.181 69.541108) (end 119.181 64.379) (width 0.2) (layer "B.Cu") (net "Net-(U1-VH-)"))
 (segment (start 124.6 76.926968) (end 119.196968 82.33) (width 0.2) (layer "F.Cu") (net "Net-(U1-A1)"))
 (segment (start 119.196968 82.33) (end 118.85 82.33) (width 0.2) (layer "F.Cu") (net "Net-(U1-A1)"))
 (segment (start 119.824999 82.33) (end 120.126 82.631001) (width 0.2) (layer "F.Cu") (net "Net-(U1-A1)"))
 (segment (start 118.85 82.33) (end 119.824999 82.33) (width 0.2) (layer "F.Cu") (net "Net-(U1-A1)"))
 (segment (start 120.126 87.674) (end 118.85 88.95) (width 0.2) (layer "F.Cu") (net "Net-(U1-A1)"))
 (segment (start 124.6 72.4) (end 124.6 76.926968) (width 0.2) (layer "F.Cu") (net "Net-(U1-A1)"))
 (segment (start 120.126 82.631001) (end 120.126 87.674) (width 0.2) (layer "F.Cu") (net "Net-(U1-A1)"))
 (segment (start 124.6 65.68) (end 124.6 72.4) (width 0.2) (layer "B.Cu") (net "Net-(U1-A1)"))
 (segment (start 123.95 87.8) (end 123.95 86.75) (width 0.2) (layer "F.Cu") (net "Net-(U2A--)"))
 (segment (start 120.2 80.4) (end 119.51 80.4) (width 0.2) (layer "F.Cu") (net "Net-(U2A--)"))
 (segment (start 119.51 80.4) (end 118.85 81.06) (width 0.2) (layer "F.Cu") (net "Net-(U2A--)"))
 (segment (start 123.95 86.75) (end 122 84.8) (width 0.2) (layer "F.Cu") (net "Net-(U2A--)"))
 (via (at 120.2 80.4) (size 0.6) (drill 0.3) (layers "F.Cu" "B.Cu") (capping no) (covering (front no) (back no))
  (plugging (front no) (back no)) (filling no) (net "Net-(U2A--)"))
 (via (at 122 84.8) (size 0.6) (drill 0.3) (layers "F.Cu" "B.Cu") (capping no) (covering (front no) (back no))
  (plugging (front no) (back no)) (filling no) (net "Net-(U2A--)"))
 (segment (start 122 82.2) (end 120.2 80.4) (width 0.2) (layer "B.Cu") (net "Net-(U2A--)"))
 (segment (start 122 84.8) (end 122 82.2) (width 0.2) (layer "B.Cu") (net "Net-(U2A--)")))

